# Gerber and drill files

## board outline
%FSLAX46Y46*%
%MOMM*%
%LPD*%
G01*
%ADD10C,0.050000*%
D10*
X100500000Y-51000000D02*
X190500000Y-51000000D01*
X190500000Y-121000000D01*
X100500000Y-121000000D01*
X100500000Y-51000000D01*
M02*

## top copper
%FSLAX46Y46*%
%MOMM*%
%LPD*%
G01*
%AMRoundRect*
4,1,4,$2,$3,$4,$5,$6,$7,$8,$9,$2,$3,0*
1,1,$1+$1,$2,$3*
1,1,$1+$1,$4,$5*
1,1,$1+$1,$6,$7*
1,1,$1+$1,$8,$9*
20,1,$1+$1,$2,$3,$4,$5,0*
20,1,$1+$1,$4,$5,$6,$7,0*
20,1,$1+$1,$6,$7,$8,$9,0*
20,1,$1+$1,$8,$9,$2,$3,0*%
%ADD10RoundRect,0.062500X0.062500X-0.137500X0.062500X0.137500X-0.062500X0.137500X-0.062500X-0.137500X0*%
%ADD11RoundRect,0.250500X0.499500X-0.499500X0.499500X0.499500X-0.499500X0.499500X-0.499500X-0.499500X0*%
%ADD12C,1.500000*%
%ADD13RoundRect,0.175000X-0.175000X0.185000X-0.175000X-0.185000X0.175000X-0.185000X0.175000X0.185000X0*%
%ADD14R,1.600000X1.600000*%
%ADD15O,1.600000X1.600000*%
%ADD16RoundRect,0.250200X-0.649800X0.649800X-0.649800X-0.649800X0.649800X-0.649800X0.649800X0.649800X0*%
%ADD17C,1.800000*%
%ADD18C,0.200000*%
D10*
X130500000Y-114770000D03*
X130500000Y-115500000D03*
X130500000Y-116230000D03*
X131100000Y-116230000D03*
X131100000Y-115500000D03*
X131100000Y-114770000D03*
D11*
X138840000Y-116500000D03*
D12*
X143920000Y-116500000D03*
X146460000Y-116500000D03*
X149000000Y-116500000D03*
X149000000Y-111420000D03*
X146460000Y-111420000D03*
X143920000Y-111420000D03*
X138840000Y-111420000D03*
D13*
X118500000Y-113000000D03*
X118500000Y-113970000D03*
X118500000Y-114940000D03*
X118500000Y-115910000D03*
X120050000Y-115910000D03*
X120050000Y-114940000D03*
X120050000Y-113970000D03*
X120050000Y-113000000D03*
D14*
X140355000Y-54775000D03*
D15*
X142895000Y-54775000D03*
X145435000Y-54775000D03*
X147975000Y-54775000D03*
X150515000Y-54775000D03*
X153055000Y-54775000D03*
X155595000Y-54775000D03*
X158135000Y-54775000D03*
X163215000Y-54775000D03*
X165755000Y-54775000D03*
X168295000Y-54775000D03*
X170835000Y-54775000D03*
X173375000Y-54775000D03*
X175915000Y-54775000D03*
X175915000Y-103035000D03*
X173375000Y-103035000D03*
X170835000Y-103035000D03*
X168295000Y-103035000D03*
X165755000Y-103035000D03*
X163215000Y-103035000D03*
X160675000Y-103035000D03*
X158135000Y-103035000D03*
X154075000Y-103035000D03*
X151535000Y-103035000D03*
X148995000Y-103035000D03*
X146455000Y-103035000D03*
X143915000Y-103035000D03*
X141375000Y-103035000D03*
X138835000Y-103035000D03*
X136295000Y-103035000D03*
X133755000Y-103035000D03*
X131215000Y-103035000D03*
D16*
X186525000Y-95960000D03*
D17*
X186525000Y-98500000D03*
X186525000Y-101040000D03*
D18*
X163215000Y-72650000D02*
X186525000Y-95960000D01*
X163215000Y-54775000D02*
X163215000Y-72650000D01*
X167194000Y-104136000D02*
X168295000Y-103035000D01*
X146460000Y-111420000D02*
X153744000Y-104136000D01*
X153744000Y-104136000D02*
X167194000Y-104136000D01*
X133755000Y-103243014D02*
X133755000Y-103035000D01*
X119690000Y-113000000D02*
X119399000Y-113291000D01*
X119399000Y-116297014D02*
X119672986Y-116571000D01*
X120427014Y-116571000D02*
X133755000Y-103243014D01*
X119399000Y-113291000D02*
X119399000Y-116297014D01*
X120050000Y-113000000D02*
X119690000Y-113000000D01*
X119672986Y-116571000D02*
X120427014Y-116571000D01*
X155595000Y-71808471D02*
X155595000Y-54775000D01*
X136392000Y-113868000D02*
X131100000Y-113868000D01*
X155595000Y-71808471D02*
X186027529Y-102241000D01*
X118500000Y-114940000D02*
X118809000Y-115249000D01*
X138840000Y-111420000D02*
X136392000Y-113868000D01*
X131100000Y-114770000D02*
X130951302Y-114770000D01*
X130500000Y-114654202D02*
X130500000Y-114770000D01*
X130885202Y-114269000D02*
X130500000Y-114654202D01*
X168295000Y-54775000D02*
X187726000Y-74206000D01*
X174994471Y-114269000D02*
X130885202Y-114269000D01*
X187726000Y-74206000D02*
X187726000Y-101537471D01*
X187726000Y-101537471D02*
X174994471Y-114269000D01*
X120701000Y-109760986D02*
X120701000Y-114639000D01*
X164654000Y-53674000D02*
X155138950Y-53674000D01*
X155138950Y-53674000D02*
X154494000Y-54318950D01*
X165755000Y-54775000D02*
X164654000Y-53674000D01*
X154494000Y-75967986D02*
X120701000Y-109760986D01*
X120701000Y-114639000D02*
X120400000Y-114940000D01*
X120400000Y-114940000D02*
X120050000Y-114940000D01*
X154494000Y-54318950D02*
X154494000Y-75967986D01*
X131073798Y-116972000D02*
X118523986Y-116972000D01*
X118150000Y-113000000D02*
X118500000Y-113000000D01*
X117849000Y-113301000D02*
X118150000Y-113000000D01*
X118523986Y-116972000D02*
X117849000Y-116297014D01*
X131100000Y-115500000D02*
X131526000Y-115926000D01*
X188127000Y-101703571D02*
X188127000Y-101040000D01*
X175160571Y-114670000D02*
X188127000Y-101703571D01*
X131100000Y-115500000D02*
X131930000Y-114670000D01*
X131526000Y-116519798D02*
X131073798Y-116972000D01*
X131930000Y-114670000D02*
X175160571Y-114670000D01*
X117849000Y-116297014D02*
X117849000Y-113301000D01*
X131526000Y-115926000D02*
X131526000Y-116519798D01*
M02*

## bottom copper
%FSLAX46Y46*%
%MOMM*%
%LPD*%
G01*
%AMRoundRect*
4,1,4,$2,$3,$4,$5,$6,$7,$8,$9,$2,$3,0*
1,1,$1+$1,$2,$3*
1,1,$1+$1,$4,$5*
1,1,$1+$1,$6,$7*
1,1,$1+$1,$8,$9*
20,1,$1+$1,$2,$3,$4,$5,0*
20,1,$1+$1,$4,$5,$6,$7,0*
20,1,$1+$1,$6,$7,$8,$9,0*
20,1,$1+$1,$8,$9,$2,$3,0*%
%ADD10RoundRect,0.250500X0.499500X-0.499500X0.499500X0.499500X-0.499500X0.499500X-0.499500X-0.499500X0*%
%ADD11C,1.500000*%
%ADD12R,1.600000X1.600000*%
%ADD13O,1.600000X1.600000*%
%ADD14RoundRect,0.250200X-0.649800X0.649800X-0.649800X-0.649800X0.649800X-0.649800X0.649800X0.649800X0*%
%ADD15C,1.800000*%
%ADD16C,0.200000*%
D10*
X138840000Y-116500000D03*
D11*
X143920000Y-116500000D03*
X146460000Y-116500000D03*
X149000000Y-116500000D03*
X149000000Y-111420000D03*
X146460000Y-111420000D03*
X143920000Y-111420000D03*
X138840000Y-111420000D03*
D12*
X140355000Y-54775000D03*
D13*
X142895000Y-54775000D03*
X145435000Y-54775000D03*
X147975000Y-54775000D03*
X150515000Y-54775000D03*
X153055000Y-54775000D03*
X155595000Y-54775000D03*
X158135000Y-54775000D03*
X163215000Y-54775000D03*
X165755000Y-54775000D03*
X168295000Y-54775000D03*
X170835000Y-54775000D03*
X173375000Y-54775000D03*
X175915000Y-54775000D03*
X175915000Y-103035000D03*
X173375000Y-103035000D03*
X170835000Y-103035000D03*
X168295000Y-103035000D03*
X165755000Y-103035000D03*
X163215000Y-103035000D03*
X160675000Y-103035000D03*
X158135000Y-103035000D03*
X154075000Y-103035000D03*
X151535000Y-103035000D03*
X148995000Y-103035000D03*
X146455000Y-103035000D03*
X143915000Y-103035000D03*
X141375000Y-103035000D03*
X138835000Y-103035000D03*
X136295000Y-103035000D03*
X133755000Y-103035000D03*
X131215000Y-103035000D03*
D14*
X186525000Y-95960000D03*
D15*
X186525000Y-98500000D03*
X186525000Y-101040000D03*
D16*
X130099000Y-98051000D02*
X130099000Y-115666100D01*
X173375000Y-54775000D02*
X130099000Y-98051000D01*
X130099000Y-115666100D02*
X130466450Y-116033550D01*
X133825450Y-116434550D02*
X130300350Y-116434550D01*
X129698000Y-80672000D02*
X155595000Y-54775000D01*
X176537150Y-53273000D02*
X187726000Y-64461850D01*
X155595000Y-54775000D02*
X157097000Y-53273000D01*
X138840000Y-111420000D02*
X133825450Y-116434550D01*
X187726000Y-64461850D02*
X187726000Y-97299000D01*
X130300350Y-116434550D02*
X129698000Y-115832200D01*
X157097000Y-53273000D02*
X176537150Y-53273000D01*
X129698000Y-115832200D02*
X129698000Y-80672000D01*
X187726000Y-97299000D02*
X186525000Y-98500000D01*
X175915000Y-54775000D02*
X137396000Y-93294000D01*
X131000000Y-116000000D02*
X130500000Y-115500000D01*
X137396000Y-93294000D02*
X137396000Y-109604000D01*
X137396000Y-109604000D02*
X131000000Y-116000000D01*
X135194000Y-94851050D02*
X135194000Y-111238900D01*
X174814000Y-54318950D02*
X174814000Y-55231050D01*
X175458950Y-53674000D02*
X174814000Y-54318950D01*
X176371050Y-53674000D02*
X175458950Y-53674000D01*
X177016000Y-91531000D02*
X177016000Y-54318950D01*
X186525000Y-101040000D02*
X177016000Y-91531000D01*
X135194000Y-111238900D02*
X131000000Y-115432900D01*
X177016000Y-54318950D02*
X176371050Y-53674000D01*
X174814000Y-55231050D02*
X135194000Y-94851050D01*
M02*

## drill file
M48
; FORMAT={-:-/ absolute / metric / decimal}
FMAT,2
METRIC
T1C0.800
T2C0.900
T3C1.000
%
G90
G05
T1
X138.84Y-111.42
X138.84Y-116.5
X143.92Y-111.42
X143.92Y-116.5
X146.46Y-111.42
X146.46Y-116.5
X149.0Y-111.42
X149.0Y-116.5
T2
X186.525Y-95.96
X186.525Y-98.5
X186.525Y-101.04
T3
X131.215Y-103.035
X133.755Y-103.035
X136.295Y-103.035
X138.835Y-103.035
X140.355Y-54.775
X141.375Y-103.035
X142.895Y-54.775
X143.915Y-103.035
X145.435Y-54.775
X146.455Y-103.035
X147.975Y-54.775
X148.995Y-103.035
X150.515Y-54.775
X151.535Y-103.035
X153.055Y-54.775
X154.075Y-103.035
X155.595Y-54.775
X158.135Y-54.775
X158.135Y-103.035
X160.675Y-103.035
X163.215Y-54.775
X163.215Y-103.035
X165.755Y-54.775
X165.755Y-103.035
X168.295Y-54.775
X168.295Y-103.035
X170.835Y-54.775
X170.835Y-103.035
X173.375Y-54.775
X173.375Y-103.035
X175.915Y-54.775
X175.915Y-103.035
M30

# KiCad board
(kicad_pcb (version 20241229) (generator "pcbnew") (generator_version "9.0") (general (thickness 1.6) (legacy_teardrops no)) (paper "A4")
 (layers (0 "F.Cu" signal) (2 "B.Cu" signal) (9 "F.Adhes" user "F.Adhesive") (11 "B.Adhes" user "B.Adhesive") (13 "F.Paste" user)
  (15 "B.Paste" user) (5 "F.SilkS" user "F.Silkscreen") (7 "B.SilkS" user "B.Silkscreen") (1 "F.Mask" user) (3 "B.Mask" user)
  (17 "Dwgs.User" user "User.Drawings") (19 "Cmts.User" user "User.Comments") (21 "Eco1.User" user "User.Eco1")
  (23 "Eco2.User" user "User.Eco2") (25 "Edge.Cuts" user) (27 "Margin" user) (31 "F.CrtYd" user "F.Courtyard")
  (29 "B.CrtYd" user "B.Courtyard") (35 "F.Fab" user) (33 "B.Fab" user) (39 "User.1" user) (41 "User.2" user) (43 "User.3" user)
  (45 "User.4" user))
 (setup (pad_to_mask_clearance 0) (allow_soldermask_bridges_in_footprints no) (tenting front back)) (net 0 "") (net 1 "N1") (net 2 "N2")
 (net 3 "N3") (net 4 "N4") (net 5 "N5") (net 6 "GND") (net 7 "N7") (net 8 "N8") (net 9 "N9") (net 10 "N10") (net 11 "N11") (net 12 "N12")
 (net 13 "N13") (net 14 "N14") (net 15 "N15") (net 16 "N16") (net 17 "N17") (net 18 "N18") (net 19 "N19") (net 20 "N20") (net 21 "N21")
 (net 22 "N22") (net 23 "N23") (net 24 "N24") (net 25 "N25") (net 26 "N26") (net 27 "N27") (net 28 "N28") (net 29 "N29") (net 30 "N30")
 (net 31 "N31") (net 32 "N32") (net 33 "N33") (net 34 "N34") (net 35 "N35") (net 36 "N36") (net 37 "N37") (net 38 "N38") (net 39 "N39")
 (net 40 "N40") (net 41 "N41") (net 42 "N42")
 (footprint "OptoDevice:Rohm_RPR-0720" (layer "F.Cu") (at 130.8 115.5)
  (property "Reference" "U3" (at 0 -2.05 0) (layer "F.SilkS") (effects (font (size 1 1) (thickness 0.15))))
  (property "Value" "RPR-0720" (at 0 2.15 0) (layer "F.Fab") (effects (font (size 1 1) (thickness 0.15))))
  (pad "1" smd roundrect (at -0.3 -0.73 90) (size 0.4 0.25) (layers "F.Cu" "F.Mask" "F.Paste") (roundrect_rratio 0.25) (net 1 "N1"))
  (pad "2" smd roundrect (at -0.3 0 90) (size 0.4 0.25) (layers "F.Cu" "F.Mask" "F.Paste") (roundrect_rratio 0.25) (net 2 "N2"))
  (pad "3" smd roundrect (at -0.3 0.73 90) (size 0.4 0.25) (layers "F.Cu" "F.Mask" "F.Paste") (roundrect_rratio 0.25) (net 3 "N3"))
  (pad "4" smd roundrect (at 0.3 0.73 90) (size 0.4 0.25) (layers "F.Cu" "F.Mask" "F.Paste") (roundrect_rratio 0.25) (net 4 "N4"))
  (pad "5" smd roundrect (at 0.3 0 90) (size 0.4 0.25) (layers "F.Cu" "F.Mask" "F.Paste") (roundrect_rratio 0.25) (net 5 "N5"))
  (pad "6" smd roundrect (at 0.3 -0.73 90) (size 0.4 0.25) (layers "F.Cu" "F.Mask" "F.Paste") (roundrect_rratio 0.25) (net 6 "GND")))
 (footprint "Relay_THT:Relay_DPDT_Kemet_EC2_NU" (layer "F.Cu") (at 138.84 116.5 90)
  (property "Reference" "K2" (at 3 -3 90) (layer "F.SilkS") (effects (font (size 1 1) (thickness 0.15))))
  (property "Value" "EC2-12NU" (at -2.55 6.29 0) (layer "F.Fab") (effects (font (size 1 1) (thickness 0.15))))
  (pad "1" thru_hole roundrect (at 0 0 90) (size 1.5 1.5) (drill 0.8) (layers "*.Cu" "*.Mask") (remove_unused_layers no)
   (roundrect_rratio 0.167) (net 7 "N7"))
  (pad "3" thru_hole circle (at 0 5.08 90) (size 1.5 1.5) (drill 0.8) (layers "*.Cu" "*.Mask") (remove_unused_layers no) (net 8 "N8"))
  (pad "4" thru_hole circle (at 0 7.62 90) (size 1.5 1.5) (drill 0.8) (layers "*.Cu" "*.Mask") (remove_unused_layers no) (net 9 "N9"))
  (pad "5" thru_hole circle (at 0 10.16 90) (size 1.5 1.5) (drill 0.8) (layers "*.Cu" "*.Mask") (remove_unused_layers no) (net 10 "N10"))
  (pad "8" thru_hole circle (at 5.08 10.16 90) (size 1.5 1.5) (drill 0.8) (layers "*.Cu" "*.Mask") (remove_unused_layers no) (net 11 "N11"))
  (pad "9" thru_hole circle (at 5.08 7.62 90) (size 1.5 1.5) (drill 0.8) (layers "*.Cu" "*.Mask") (remove_unused_layers no) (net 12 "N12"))
  (pad "10" thru_hole circle (at 5.08 5.08 90) (size 1.5 1.5) (drill 0.8) (layers "*.Cu" "*.Mask") (remove_unused_layers no) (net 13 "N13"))
  (pad "12" thru_hole circle (at 5.08 0 90) (size 1.5 1.5) (drill 0.8) (layers "*.Cu" "*.Mask") (remove_unused_layers no) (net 6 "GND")))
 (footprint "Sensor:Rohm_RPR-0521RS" (layer "F.Cu") (at 119.275 114.455)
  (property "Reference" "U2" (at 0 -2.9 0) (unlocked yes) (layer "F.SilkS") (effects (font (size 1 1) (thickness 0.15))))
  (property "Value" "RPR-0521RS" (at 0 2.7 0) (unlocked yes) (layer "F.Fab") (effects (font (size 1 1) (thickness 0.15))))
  (pad "1" smd roundrect (at -0.775 -1.455 270) (size 0.72 0.7) (layers "F.Cu" "F.Mask" "F.Paste") (roundrect_rratio 0.25) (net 5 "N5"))
  (pad "2" smd roundrect (at -0.775 -0.485 270) (size 0.72 0.7) (layers "F.Cu" "F.Mask" "F.Paste") (roundrect_rratio 0.25) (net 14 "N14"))
  (pad "3" smd roundrect (at -0.775 0.485 270) (size 0.72 0.7) (layers "F.Cu" "F.Mask" "F.Paste") (roundrect_rratio 0.25) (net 6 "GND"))
  (pad "4" smd roundrect (at -0.775 1.455 270) (size 0.72 0.7) (layers "F.Cu" "F.Mask" "F.Paste") (roundrect_rratio 0.25) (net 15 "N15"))
  (pad "5" smd roundrect (at 0.775 1.455 270) (size 0.72 0.7) (layers "F.Cu" "F.Mask" "F.Paste") (roundrect_rratio 0.25) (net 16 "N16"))
  (pad "6" smd roundrect (at 0.775 0.485 270) (size 0.72 0.7) (layers "F.Cu" "F.Mask" "F.Paste") (roundrect_rratio 0.25) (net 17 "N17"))
  (pad "7" smd roundrect (at 0.775 -0.485 270) (size 0.72 0.7) (layers "F.Cu" "F.Mask" "F.Paste") (roundrect_rratio 0.25) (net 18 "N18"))
  (pad "8" smd roundrect (at 0.775 -1.455 270) (size 0.72 0.7) (layers "F.Cu" "F.Mask" "F.Paste") (roundrect_rratio 0.25) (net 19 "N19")))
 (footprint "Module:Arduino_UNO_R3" (layer "F.Cu") (at 140.355 54.775)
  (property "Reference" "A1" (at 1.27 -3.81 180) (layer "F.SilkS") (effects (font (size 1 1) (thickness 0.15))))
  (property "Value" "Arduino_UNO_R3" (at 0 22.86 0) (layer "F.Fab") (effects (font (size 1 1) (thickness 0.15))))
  (pad "1" thru_hole rect (at 0 0 90) (size 1.6 1.6) (drill 1) (layers "*.Cu" "*.Mask") (remove_unused_layers no) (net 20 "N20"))
  (pad "2" thru_hole oval (at 2.54 0 90) (size 1.6 1.6) (drill 1) (layers "*.Cu" "*.Mask") (remove_unused_layers no) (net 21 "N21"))
  (pad "3" thru_hole oval (at 5.08 0 90) (size 1.6 1.6) (drill 1) (layers "*.Cu" "*.Mask") (remove_unused_layers no) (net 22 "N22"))
  (pad "4" thru_hole oval (at 7.62 0 90) (size 1.6 1.6) (drill 1) (layers "*.Cu" "*.Mask") (remove_unused_layers no) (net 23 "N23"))
  (pad "5" thru_hole oval (at 10.16 0 90) (size 1.6 1.6) (drill 1) (layers "*.Cu" "*.Mask") (remove_unused_layers no) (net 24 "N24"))
  (pad "6" thru_hole oval (at 12.7 0 90) (size 1.6 1.6) (drill 1) (layers "*.Cu" "*.Mask") (remove_unused_layers no) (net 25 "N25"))
  (pad "7" thru_hole oval (at 15.24 0 90) (size 1.6 1.6) (drill 1) (layers "*.Cu" "*.Mask") (remove_unused_layers no) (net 6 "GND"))
  (pad "8" thru_hole oval (at 17.78 0 90) (size 1.6 1.6) (drill 1) (layers "*.Cu" "*.Mask") (remove_unused_layers no) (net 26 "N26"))
  (pad "9" thru_hole oval (at 22.86 0 90) (size 1.6 1.6) (drill 1) (layers "*.Cu" "*.Mask") (remove_unused_layers no) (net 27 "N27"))
  (pad "10" thru_hole oval (at 25.4 0 90) (size 1.6 1.6) (drill 1) (layers "*.Cu" "*.Mask") (remove_unused_layers no) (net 17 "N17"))
  (pad "11" thru_hole oval (at 27.94 0 90) (size 1.6 1.6) (drill 1) (layers "*.Cu" "*.Mask") (remove_unused_layers no) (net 1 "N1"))
  (pad "12" thru_hole oval (at 30.48 0 90) (size 1.6 1.6) (drill 1) (layers "*.Cu" "*.Mask") (remove_unused_layers no) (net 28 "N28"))
  (pad "13" thru_hole oval (at 33.02 0 90) (size 1.6 1.6) (drill 1) (layers "*.Cu" "*.Mask") (remove_unused_layers no) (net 3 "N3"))
  (pad "14" thru_hole oval (at 35.56 0 90) (size 1.6 1.6) (drill 1) (layers "*.Cu" "*.Mask") (remove_unused_layers no) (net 2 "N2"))
  (pad "15" thru_hole oval (at 35.56 48.26 90) (size 1.6 1.6) (drill 1) (layers "*.Cu" "*.Mask") (remove_unused_layers no) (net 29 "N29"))
  (pad "16" thru_hole oval (at 33.02 48.26 90) (size 1.6 1.6) (drill 1) (layers "*.Cu" "*.Mask") (remove_unused_layers no) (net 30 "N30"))
  (pad "17" thru_hole oval (at 30.48 48.26 90) (size 1.6 1.6) (drill 1) (layers "*.Cu" "*.Mask") (remove_unused_layers no) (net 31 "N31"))
  (pad "18" thru_hole oval (at 27.94 48.26 90) (size 1.6 1.6) (drill 1) (layers "*.Cu" "*.Mask") (remove_unused_layers no) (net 12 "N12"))
  (pad "19" thru_hole oval (at 25.4 48.26 90) (size 1.6 1.6) (drill 1) (layers "*.Cu" "*.Mask") (remove_unused_layers no) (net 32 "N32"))
  (pad "20" thru_hole oval (at 22.86 48.26 90) (size 1.6 1.6) (drill 1) (layers "*.Cu" "*.Mask") (remove_unused_layers no) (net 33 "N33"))
  (pad "21" thru_hole oval (at 20.32 48.26 90) (size 1.6 1.6) (drill 1) (layers "*.Cu" "*.Mask") (remove_unused_layers no) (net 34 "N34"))
  (pad "22" thru_hole oval (at 17.78 48.26 90) (size 1.6 1.6) (drill 1) (layers "*.Cu" "*.Mask") (remove_unused_layers no) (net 9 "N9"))
  (pad "23" thru_hole oval (at 13.72 48.26 90) (size 1.6 1.6) (drill 1) (layers "*.Cu" "*.Mask") (remove_unused_layers no) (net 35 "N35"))
  (pad "24" thru_hole oval (at 11.18 48.26 90) (size 1.6 1.6) (drill 1) (layers "*.Cu" "*.Mask") (remove_unused_layers no) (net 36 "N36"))
  (pad "25" thru_hole oval (at 8.64 48.26 90) (size 1.6 1.6) (drill 1) (layers "*.Cu" "*.Mask") (remove_unused_layers no) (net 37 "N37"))
  (pad "26" thru_hole oval (at 6.1 48.26 90) (size 1.6 1.6) (drill 1) (layers "*.Cu" "*.Mask") (remove_unused_layers no) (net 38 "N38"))
  (pad "27" thru_hole oval (at 3.56 48.26 90) (size 1.6 1.6) (drill 1) (layers "*.Cu" "*.Mask") (remove_unused_layers no) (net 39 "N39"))
  (pad "28" thru_hole oval (at 1.02 48.26 90) (size 1.6 1.6) (drill 1) (layers "*.Cu" "*.Mask") (remove_unused_layers no) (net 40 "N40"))
  (pad "29" thru_hole oval (at -1.52 48.26 90) (size 1.6 1.6) (drill 1) (layers "*.Cu" "*.Mask") (remove_unused_layers no) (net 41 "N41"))
  (pad "30" thru_hole oval (at -4.06 48.26 90) (size 1.6 1.6) (drill 1) (layers "*.Cu" "*.Mask") (remove_unused_layers no) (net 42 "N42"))
  (pad "31" thru_hole oval (at -6.6 48.26 90) (size 1.6 1.6) (drill 1) (layers "*.Cu" "*.Mask") (remove_unused_layers no) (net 19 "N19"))
  (pad "32" thru_hole oval (at -9.14 48.26 90) (size 1.6 1.6) (drill 1) (layers "*.Cu" "*.Mask") (remove_unused_layers no) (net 14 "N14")))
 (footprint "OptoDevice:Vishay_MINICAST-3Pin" (layer "F.Cu") (at 186.525 95.96 -90)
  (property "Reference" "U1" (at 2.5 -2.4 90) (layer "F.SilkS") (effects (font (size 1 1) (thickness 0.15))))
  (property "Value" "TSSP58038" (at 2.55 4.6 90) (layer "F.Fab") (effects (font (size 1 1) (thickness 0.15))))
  (pad "1" thru_hole roundrect (at 0 0 270) (size 1.8 1.8) (drill 0.9) (layers "*.Cu" "*.Mask") (remove_unused_layers no)
   (roundrect_rratio 0.139) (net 27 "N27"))
  (pad "2" thru_hole circle (at 2.54 0 270) (size 1.8 1.8) (drill 0.9) (layers "*.Cu" "*.Mask") (remove_unused_layers no) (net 6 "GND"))
  (pad "3" thru_hole circle (at 5.08 0 270) (size 1.8 1.8) (drill 0.9) (layers "*.Cu" "*.Mask") (remove_unused_layers no) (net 5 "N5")))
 (gr_rect (start 100.5 51) (end 190.5 121) (stroke (width 0.05) (type default)) (fill no) (layer "Edge.Cuts"))
 (segment (start 163.215 72.65) (end 186.525 95.96) (width 0.2) (layer "F.Cu") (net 27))
 (segment (start 163.215 54.775) (end 163.215 72.65) (width 0.2) (layer "F.Cu") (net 27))
 (segment (start 167.194 104.136) (end 168.295 103.035) (width 0.2) (layer "F.Cu") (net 12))
 (segment (start 146.46 111.42) (end 153.744 104.136) (width 0.2) (layer "F.Cu") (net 12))
 (segment (start 153.744 104.136) (end 167.194 104.136) (width 0.2) (layer "F.Cu") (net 12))
 (segment (start 130.099 98.051) (end 130.099 115.6661) (width 0.2) (layer "B.Cu") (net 3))
 (segment (start 173.375 54.775) (end 130.099 98.051) (width 0.2) (layer "B.Cu") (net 3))
 (segment (start 130.099 115.6661) (end 130.46645 116.03355) (width 0.2) (layer "B.Cu") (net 3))
 (segment (start 133.755 103.243014) (end 133.755 103.035) (width 0.2) (layer "F.Cu") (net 19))
 (segment (start 119.69 113) (end 119.399 113.291) (width 0.2) (layer "F.Cu") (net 19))
 (segment (start 119.399 116.297014) (end 119.672986 116.571) (width 0.2) (layer "F.Cu") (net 19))
 (segment (start 120.427014 116.571) (end 133.755 103.243014) (width 0.2) (layer "F.Cu") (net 19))
 (segment (start 119.399 113.291) (end 119.399 116.297014) (width 0.2) (layer "F.Cu") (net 19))
 (segment (start 120.05 113) (end 119.69 113) (width 0.2) (layer "F.Cu") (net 19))
 (segment (start 119.672986 116.571) (end 120.427014 116.571) (width 0.2) (layer "F.Cu") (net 19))
 (segment (start 155.595 71.808471) (end 155.595 54.775) (width 0.2) (layer "F.Cu") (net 6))
 (segment (start 136.392 113.868) (end 131.1 113.868) (width 0.2) (layer "F.Cu") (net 6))
 (segment (start 155.595 71.808471) (end 186.027529 102.241) (width 0.2) (layer "F.Cu") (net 6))
 (segment (start 118.5 114.94) (end 118.809 115.249) (width 0.2) (layer "F.Cu") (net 6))
 (segment (start 138.84 111.42) (end 136.392 113.868) (width 0.2) (layer "F.Cu") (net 6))
 (segment (start 131.1 114.77) (end 130.951302 114.77) (width 0.2) (layer "F.Cu") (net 6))
 (segment (start 133.82545 116.43455) (end 130.30035 116.43455) (width 0.2) (layer "B.Cu") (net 6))
 (segment (start 129.698 80.672) (end 155.595 54.775) (width 0.2) (layer "B.Cu") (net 6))
 (segment (start 176.53715 53.273) (end 187.726 64.46185) (width 0.2) (layer "B.Cu") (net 6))
 (segment (start 155.595 54.775) (end 157.097 53.273) (width 0.2) (layer "B.Cu") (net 6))
 (segment (start 138.84 111.42) (end 133.82545 116.43455) (width 0.2) (layer "B.Cu") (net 6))
 (segment (start 187.726 64.46185) (end 187.726 97.299) (width 0.2) (layer "B.Cu") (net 6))
 (segment (start 130.30035 116.43455) (end 129.698 115.8322) (width 0.2) (layer "B.Cu") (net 6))
 (segment (start 157.097 53.273) (end 176.53715 53.273) (width 0.2) (layer "B.Cu") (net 6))
 (segment (start 129.698 115.8322) (end 129.698 80.672) (width 0.2) (layer "B.Cu") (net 6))
 (segment (start 187.726 97.299) (end 186.525 98.5) (width 0.2) (layer "B.Cu") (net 6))
 (segment (start 130.5 114.654202) (end 130.5 114.77) (width 0.2) (layer "F.Cu") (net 1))
 (segment (start 130.885202 114.269) (end 130.5 114.654202) (width 0.2) (layer "F.Cu") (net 1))
 (segment (start 168.295 54.775) (end 187.726 74.206) (width 0.2) (layer "F.Cu") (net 1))
 (segment (start 174.994471 114.269) (end 130.885202 114.269) (width 0.2) (layer "F.Cu") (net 1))
 (segment (start 187.726 74.206) (end 187.726 101.537471) (width 0.2) (layer "F.Cu") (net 1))
 (segment (start 187.726 101.537471) (end 174.994471 114.269) (width 0.2) (layer "F.Cu") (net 1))
 (segment (start 175.915 54.775) (end 137.396 93.294) (width 0.2) (layer "B.Cu") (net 2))
 (segment (start 131 116) (end 130.5 115.5) (width 0.2) (layer "B.Cu") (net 2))
 (segment (start 137.396 93.294) (end 137.396 109.604) (width 0.2) (layer "B.Cu") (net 2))
 (segment (start 137.396 109.604) (end 131 116) (width 0.2) (layer "B.Cu") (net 2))
 (segment (start 120.701 109.760986) (end 120.701 114.639) (width 0.2) (layer "F.Cu") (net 17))
 (segment (start 164.654 53.674) (end 155.13895 53.674) (width 0.2) (layer "F.Cu") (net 17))
 (segment (start 155.13895 53.674) (end 154.494 54.31895) (width 0.2) (layer "F.Cu") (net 17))
 (segment (start 165.755 54.775) (end 164.654 53.674) (width 0.2) (layer "F.Cu") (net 17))
 (segment (start 154.494 75.967986) (end 120.701 109.760986) (width 0.2) (layer "F.Cu") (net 17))
 (segment (start 120.701 114.639) (end 120.4 114.94) (width 0.2) (layer "F.Cu") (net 17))
 (segment (start 120.4 114.94) (end 120.05 114.94) (width 0.2) (layer "F.Cu") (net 17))
 (segment (start 154.494 54.31895) (end 154.494 75.967986) (width 0.2) (layer "F.Cu") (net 17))
 (segment (start 131.073798 116.972) (end 118.523986 116.972) (width 0.2) (layer "F.Cu") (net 5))
 (segment (start 118.15 113) (end 118.5 113) (width 0.2) (layer "F.Cu") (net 5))
 (segment (start 117.849 113.301) (end 118.15 113) (width 0.2) (layer "F.Cu") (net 5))
 (segment (start 118.523986 116.972) (end 117.849 116.297014) (width 0.2) (layer "F.Cu") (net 5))
 (segment (start 131.1 115.5) (end 131.526 115.926) (width 0.2) (layer "F.Cu") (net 5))
 (segment (start 188.127 101.703571) (end 188.127 101.04) (width 0.2) (layer "F.Cu") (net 5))
 (segment (start 175.160571 114.67) (end 188.127 101.703571) (width 0.2) (layer "F.Cu") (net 5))
 (segment (start 131.1 115.5) (end 131.93 114.67) (width 0.2) (layer "F.Cu") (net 5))
 (segment (start 131.526 116.519798) (end 131.073798 116.972) (width 0.2) (layer "F.Cu") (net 5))
 (segment (start 131.93 114.67) (end 175.160571 114.67) (width 0.2) (layer "F.Cu") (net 5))
 (segment (start 117.849 116.297014) (end 117.849 113.301) (width 0.2) (layer "F.Cu") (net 5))
 (segment (start 131.526 115.926) (end 131.526 116.519798) (width 0.2) (layer "F.Cu") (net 5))
 (segment (start 135.194 94.85105) (end 135.194 111.2389) (width 0.2) (layer "B.Cu") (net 5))
 (segment (start 174.814 54.31895) (end 174.814 55.23105) (width 0.2) (layer "B.Cu") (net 5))
 (segment (start 175.45895 53.674) (end 174.814 54.31895) (width 0.2) (layer "B.Cu") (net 5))
 (segment (start 176.37105 53.674) (end 175.45895 53.674) (width 0.2) (layer "B.Cu") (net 5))
 (segment (start 177.016 91.531) (end 177.016 54.31895) (width 0.2) (layer "B.Cu") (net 5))
 (segment (start 186.525 101.04) (end 177.016 91.531) (width 0.2) (layer "B.Cu") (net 5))
 (segment (start 135.194 111.2389) (end 131 115.4329) (width 0.2) (layer "B.Cu") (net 5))
 (segment (start 177.016 54.31895) (end 176.37105 53.674) (width 0.2) (layer "B.Cu") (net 5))
 (segment (start 174.814 55.23105) (end 135.194 94.85105) (width 0.2) (layer "B.Cu") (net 5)))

